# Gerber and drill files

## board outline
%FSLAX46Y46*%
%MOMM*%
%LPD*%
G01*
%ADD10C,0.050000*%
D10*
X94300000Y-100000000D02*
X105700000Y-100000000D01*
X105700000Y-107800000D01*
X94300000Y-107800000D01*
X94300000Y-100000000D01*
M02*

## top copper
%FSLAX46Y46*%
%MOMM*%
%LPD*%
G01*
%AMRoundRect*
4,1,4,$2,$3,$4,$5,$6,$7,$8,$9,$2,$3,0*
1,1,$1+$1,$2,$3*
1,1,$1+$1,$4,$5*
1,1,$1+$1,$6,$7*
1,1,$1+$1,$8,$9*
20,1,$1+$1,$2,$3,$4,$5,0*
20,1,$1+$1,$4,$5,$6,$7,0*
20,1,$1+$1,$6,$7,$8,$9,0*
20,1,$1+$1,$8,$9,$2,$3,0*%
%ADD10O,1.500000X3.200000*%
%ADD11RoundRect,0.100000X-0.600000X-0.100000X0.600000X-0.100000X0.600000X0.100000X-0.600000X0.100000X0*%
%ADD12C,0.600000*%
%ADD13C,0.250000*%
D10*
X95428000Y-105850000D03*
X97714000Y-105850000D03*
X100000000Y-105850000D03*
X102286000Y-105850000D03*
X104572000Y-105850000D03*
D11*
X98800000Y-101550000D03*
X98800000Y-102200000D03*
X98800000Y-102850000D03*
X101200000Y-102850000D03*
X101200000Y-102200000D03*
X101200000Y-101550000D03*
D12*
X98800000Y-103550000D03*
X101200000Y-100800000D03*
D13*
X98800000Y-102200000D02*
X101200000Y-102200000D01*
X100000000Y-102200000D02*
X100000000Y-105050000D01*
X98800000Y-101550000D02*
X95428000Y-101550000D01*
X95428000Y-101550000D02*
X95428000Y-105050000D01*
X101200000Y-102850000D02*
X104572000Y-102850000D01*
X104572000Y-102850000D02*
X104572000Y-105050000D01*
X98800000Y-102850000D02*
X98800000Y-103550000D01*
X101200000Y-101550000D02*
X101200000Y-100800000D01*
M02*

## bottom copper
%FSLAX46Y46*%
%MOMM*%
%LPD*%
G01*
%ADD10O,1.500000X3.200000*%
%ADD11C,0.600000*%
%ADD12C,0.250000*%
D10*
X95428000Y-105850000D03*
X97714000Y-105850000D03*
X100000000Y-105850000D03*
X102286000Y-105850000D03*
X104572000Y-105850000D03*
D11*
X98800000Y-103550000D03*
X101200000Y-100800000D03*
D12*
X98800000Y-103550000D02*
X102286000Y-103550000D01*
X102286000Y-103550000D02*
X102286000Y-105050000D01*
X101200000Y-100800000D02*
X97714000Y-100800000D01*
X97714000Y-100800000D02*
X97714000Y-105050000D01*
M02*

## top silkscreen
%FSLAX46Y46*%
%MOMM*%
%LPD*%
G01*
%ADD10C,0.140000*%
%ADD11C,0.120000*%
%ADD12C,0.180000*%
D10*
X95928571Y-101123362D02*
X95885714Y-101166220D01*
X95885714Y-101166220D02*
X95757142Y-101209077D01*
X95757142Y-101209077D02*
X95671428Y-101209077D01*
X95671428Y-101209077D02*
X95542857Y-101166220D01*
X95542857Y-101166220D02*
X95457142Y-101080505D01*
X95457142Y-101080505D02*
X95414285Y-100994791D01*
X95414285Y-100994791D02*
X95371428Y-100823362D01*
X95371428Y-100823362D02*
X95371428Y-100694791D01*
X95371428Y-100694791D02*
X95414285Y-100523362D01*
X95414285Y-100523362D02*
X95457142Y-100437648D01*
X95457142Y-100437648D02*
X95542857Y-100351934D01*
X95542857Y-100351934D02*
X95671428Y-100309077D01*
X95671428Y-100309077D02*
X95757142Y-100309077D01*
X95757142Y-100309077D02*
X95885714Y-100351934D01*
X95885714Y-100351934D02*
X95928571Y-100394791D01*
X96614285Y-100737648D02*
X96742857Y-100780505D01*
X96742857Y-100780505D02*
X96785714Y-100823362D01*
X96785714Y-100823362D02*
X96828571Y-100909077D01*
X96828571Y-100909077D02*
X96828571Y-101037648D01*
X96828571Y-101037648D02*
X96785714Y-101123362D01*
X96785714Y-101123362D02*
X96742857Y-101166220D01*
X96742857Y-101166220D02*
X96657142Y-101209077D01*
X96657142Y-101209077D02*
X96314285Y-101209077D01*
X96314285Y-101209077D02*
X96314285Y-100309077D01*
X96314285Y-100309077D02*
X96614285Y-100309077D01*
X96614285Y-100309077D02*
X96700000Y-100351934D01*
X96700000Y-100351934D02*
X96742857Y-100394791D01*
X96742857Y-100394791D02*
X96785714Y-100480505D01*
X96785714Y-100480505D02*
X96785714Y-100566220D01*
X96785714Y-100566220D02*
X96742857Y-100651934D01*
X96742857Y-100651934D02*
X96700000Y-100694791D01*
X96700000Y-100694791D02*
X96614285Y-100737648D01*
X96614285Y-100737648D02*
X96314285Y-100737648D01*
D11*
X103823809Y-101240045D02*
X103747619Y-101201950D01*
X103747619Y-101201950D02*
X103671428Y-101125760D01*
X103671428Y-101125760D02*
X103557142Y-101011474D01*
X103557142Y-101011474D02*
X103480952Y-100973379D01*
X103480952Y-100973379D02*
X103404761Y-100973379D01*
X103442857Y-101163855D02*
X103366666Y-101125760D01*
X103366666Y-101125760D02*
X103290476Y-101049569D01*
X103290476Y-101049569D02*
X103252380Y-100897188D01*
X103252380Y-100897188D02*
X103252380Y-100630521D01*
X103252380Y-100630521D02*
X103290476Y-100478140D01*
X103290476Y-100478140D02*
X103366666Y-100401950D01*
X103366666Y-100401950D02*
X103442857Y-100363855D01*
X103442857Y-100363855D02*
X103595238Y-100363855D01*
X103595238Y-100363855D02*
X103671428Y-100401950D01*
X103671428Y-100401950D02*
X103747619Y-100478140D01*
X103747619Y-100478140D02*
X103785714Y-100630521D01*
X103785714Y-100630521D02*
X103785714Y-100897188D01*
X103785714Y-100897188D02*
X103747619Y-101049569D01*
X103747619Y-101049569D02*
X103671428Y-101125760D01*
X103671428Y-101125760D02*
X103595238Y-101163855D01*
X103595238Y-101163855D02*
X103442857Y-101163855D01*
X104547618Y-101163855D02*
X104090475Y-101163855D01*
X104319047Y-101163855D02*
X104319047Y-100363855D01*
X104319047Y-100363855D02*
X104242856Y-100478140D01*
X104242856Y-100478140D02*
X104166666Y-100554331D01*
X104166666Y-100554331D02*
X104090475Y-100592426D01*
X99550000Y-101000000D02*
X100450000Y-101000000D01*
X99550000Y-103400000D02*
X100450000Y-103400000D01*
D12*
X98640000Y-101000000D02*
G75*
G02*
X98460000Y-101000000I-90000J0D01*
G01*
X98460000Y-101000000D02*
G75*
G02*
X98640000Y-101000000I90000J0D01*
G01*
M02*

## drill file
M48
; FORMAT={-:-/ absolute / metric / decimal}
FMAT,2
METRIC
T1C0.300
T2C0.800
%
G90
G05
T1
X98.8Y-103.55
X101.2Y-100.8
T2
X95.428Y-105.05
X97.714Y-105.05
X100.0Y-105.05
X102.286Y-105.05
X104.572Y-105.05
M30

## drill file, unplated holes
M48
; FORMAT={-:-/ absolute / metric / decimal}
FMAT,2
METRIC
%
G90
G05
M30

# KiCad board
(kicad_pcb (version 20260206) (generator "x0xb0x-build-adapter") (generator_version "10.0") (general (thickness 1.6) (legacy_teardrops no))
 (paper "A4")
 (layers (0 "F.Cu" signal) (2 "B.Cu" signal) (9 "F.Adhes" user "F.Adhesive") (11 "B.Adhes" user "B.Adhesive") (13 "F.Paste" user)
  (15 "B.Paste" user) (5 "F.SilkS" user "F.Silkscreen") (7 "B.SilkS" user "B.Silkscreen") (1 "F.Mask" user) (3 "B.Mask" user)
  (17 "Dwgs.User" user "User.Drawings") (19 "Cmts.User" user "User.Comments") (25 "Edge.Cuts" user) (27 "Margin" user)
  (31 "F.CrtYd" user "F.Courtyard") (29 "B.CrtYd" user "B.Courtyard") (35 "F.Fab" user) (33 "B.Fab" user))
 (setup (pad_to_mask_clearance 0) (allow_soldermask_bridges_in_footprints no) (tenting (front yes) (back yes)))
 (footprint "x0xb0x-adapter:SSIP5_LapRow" (layer "F.Cu") (at 100.0 105.05)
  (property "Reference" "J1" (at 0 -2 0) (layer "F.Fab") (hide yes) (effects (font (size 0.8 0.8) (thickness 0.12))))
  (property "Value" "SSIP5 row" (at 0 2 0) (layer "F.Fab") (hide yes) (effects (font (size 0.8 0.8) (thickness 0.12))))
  (pad "1" thru_hole oval (at -4.572 0) (size 1.5 3.2) (drill 0.8 (offset 0 0.8)) (layers "*.Cu" "*.Mask") (remove_unused_layers no)
   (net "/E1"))
  (pad "2" thru_hole oval (at -2.286 0) (size 1.5 3.2) (drill 0.8 (offset 0 0.8)) (layers "*.Cu" "*.Mask") (remove_unused_layers no)
   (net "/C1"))
  (pad "3" thru_hole oval (at 0.000 0) (size 1.5 3.2) (drill 0.8 (offset 0 0.8)) (layers "*.Cu" "*.Mask") (remove_unused_layers no)
   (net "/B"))
  (pad "4" thru_hole oval (at 2.286 0) (size 1.5 3.2) (drill 0.8 (offset 0 0.8)) (layers "*.Cu" "*.Mask") (remove_unused_layers no)
   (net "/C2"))
  (pad "5" thru_hole oval (at 4.572 0) (size 1.5 3.2) (drill 0.8 (offset 0 0.8)) (layers "*.Cu" "*.Mask") (remove_unused_layers no)
   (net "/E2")))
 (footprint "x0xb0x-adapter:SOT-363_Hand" (layer "F.Cu") (at 100.0 102.2)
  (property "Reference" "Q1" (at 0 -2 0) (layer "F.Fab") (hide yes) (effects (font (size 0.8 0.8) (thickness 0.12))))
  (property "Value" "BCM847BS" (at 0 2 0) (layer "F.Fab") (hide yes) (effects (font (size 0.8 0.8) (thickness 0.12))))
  (fp_line (start -0.45 -1.2) (end 0.45 -1.2) (stroke (width 0.12) (type solid)) (layer "F.SilkS"))
  (fp_line (start -0.45 1.2) (end 0.45 1.2) (stroke (width 0.12) (type solid)) (layer "F.SilkS"))
  (fp_circle (center -1.45 -1.2) (end -1.33 -1.2) (stroke (width 0.12) (type solid)) (fill yes) (layer "F.SilkS"))
  (pad "1" smd roundrect (at -1.2 -0.65) (size 1.4 0.4) (layers "F.Cu" "F.Mask" "F.Paste") (roundrect_rratio 0.25) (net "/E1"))
  (pad "2" smd roundrect (at -1.2 0) (size 1.4 0.4) (layers "F.Cu" "F.Mask" "F.Paste") (roundrect_rratio 0.25) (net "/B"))
  (pad "3" smd roundrect (at -1.2 0.65) (size 1.4 0.4) (layers "F.Cu" "F.Mask" "F.Paste") (roundrect_rratio 0.25) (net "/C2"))
  (pad "4" smd roundrect (at 1.2 0.65) (size 1.4 0.4) (layers "F.Cu" "F.Mask" "F.Paste") (roundrect_rratio 0.25) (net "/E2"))
  (pad "5" smd roundrect (at 1.2 0) (size 1.4 0.4) (layers "F.Cu" "F.Mask" "F.Paste") (roundrect_rratio 0.25) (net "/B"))
  (pad "6" smd roundrect (at 1.2 -0.65) (size 1.4 0.4) (layers "F.Cu" "F.Mask" "F.Paste") (roundrect_rratio 0.25) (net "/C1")))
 (segment (start 98.8 102.2) (end 101.2 102.2) (width 0.25) (layer "F.Cu") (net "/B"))
 (segment (start 100.0 102.2) (end 100.0 105.05) (width 0.25) (layer "F.Cu") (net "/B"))
 (segment (start 98.8 101.55) (end 95.428 101.55) (width 0.25) (layer "F.Cu") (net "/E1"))
 (segment (start 95.428 101.55) (end 95.428 105.05) (width 0.25) (layer "F.Cu") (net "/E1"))
 (segment (start 101.2 102.85) (end 104.572 102.85) (width 0.25) (layer "F.Cu") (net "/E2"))
 (segment (start 104.572 102.85) (end 104.572 105.05) (width 0.25) (layer "F.Cu") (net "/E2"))
 (segment (start 98.8 102.85) (end 98.8 103.55) (width 0.25) (layer "F.Cu") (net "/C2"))
 (segment (start 98.8 103.55) (end 102.286 103.55) (width 0.25) (layer "B.Cu") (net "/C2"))
 (segment (start 102.286 103.55) (end 102.286 105.05) (width 0.25) (layer "B.Cu") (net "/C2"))
 (segment (start 101.2 101.55) (end 101.2 100.8) (width 0.25) (layer "F.Cu") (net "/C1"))
 (segment (start 101.2 100.8) (end 97.714 100.8) (width 0.25) (layer "B.Cu") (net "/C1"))
 (segment (start 97.714 100.8) (end 97.714 105.05) (width 0.25) (layer "B.Cu") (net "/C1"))
 (via (at 98.8 103.55) (size 0.6) (drill 0.3) (layers "F.Cu" "B.Cu") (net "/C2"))
 (via (at 101.2 100.8) (size 0.6) (drill 0.3) (layers "F.Cu" "B.Cu") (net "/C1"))
 (gr_rect (start 94.3 100.0) (end 105.7 107.8) (stroke (width 0.05) (type default)) (fill no) (layer "Edge.Cuts"))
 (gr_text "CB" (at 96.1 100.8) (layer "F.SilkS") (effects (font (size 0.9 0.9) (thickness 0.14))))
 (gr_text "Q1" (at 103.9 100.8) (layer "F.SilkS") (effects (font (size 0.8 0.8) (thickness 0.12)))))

